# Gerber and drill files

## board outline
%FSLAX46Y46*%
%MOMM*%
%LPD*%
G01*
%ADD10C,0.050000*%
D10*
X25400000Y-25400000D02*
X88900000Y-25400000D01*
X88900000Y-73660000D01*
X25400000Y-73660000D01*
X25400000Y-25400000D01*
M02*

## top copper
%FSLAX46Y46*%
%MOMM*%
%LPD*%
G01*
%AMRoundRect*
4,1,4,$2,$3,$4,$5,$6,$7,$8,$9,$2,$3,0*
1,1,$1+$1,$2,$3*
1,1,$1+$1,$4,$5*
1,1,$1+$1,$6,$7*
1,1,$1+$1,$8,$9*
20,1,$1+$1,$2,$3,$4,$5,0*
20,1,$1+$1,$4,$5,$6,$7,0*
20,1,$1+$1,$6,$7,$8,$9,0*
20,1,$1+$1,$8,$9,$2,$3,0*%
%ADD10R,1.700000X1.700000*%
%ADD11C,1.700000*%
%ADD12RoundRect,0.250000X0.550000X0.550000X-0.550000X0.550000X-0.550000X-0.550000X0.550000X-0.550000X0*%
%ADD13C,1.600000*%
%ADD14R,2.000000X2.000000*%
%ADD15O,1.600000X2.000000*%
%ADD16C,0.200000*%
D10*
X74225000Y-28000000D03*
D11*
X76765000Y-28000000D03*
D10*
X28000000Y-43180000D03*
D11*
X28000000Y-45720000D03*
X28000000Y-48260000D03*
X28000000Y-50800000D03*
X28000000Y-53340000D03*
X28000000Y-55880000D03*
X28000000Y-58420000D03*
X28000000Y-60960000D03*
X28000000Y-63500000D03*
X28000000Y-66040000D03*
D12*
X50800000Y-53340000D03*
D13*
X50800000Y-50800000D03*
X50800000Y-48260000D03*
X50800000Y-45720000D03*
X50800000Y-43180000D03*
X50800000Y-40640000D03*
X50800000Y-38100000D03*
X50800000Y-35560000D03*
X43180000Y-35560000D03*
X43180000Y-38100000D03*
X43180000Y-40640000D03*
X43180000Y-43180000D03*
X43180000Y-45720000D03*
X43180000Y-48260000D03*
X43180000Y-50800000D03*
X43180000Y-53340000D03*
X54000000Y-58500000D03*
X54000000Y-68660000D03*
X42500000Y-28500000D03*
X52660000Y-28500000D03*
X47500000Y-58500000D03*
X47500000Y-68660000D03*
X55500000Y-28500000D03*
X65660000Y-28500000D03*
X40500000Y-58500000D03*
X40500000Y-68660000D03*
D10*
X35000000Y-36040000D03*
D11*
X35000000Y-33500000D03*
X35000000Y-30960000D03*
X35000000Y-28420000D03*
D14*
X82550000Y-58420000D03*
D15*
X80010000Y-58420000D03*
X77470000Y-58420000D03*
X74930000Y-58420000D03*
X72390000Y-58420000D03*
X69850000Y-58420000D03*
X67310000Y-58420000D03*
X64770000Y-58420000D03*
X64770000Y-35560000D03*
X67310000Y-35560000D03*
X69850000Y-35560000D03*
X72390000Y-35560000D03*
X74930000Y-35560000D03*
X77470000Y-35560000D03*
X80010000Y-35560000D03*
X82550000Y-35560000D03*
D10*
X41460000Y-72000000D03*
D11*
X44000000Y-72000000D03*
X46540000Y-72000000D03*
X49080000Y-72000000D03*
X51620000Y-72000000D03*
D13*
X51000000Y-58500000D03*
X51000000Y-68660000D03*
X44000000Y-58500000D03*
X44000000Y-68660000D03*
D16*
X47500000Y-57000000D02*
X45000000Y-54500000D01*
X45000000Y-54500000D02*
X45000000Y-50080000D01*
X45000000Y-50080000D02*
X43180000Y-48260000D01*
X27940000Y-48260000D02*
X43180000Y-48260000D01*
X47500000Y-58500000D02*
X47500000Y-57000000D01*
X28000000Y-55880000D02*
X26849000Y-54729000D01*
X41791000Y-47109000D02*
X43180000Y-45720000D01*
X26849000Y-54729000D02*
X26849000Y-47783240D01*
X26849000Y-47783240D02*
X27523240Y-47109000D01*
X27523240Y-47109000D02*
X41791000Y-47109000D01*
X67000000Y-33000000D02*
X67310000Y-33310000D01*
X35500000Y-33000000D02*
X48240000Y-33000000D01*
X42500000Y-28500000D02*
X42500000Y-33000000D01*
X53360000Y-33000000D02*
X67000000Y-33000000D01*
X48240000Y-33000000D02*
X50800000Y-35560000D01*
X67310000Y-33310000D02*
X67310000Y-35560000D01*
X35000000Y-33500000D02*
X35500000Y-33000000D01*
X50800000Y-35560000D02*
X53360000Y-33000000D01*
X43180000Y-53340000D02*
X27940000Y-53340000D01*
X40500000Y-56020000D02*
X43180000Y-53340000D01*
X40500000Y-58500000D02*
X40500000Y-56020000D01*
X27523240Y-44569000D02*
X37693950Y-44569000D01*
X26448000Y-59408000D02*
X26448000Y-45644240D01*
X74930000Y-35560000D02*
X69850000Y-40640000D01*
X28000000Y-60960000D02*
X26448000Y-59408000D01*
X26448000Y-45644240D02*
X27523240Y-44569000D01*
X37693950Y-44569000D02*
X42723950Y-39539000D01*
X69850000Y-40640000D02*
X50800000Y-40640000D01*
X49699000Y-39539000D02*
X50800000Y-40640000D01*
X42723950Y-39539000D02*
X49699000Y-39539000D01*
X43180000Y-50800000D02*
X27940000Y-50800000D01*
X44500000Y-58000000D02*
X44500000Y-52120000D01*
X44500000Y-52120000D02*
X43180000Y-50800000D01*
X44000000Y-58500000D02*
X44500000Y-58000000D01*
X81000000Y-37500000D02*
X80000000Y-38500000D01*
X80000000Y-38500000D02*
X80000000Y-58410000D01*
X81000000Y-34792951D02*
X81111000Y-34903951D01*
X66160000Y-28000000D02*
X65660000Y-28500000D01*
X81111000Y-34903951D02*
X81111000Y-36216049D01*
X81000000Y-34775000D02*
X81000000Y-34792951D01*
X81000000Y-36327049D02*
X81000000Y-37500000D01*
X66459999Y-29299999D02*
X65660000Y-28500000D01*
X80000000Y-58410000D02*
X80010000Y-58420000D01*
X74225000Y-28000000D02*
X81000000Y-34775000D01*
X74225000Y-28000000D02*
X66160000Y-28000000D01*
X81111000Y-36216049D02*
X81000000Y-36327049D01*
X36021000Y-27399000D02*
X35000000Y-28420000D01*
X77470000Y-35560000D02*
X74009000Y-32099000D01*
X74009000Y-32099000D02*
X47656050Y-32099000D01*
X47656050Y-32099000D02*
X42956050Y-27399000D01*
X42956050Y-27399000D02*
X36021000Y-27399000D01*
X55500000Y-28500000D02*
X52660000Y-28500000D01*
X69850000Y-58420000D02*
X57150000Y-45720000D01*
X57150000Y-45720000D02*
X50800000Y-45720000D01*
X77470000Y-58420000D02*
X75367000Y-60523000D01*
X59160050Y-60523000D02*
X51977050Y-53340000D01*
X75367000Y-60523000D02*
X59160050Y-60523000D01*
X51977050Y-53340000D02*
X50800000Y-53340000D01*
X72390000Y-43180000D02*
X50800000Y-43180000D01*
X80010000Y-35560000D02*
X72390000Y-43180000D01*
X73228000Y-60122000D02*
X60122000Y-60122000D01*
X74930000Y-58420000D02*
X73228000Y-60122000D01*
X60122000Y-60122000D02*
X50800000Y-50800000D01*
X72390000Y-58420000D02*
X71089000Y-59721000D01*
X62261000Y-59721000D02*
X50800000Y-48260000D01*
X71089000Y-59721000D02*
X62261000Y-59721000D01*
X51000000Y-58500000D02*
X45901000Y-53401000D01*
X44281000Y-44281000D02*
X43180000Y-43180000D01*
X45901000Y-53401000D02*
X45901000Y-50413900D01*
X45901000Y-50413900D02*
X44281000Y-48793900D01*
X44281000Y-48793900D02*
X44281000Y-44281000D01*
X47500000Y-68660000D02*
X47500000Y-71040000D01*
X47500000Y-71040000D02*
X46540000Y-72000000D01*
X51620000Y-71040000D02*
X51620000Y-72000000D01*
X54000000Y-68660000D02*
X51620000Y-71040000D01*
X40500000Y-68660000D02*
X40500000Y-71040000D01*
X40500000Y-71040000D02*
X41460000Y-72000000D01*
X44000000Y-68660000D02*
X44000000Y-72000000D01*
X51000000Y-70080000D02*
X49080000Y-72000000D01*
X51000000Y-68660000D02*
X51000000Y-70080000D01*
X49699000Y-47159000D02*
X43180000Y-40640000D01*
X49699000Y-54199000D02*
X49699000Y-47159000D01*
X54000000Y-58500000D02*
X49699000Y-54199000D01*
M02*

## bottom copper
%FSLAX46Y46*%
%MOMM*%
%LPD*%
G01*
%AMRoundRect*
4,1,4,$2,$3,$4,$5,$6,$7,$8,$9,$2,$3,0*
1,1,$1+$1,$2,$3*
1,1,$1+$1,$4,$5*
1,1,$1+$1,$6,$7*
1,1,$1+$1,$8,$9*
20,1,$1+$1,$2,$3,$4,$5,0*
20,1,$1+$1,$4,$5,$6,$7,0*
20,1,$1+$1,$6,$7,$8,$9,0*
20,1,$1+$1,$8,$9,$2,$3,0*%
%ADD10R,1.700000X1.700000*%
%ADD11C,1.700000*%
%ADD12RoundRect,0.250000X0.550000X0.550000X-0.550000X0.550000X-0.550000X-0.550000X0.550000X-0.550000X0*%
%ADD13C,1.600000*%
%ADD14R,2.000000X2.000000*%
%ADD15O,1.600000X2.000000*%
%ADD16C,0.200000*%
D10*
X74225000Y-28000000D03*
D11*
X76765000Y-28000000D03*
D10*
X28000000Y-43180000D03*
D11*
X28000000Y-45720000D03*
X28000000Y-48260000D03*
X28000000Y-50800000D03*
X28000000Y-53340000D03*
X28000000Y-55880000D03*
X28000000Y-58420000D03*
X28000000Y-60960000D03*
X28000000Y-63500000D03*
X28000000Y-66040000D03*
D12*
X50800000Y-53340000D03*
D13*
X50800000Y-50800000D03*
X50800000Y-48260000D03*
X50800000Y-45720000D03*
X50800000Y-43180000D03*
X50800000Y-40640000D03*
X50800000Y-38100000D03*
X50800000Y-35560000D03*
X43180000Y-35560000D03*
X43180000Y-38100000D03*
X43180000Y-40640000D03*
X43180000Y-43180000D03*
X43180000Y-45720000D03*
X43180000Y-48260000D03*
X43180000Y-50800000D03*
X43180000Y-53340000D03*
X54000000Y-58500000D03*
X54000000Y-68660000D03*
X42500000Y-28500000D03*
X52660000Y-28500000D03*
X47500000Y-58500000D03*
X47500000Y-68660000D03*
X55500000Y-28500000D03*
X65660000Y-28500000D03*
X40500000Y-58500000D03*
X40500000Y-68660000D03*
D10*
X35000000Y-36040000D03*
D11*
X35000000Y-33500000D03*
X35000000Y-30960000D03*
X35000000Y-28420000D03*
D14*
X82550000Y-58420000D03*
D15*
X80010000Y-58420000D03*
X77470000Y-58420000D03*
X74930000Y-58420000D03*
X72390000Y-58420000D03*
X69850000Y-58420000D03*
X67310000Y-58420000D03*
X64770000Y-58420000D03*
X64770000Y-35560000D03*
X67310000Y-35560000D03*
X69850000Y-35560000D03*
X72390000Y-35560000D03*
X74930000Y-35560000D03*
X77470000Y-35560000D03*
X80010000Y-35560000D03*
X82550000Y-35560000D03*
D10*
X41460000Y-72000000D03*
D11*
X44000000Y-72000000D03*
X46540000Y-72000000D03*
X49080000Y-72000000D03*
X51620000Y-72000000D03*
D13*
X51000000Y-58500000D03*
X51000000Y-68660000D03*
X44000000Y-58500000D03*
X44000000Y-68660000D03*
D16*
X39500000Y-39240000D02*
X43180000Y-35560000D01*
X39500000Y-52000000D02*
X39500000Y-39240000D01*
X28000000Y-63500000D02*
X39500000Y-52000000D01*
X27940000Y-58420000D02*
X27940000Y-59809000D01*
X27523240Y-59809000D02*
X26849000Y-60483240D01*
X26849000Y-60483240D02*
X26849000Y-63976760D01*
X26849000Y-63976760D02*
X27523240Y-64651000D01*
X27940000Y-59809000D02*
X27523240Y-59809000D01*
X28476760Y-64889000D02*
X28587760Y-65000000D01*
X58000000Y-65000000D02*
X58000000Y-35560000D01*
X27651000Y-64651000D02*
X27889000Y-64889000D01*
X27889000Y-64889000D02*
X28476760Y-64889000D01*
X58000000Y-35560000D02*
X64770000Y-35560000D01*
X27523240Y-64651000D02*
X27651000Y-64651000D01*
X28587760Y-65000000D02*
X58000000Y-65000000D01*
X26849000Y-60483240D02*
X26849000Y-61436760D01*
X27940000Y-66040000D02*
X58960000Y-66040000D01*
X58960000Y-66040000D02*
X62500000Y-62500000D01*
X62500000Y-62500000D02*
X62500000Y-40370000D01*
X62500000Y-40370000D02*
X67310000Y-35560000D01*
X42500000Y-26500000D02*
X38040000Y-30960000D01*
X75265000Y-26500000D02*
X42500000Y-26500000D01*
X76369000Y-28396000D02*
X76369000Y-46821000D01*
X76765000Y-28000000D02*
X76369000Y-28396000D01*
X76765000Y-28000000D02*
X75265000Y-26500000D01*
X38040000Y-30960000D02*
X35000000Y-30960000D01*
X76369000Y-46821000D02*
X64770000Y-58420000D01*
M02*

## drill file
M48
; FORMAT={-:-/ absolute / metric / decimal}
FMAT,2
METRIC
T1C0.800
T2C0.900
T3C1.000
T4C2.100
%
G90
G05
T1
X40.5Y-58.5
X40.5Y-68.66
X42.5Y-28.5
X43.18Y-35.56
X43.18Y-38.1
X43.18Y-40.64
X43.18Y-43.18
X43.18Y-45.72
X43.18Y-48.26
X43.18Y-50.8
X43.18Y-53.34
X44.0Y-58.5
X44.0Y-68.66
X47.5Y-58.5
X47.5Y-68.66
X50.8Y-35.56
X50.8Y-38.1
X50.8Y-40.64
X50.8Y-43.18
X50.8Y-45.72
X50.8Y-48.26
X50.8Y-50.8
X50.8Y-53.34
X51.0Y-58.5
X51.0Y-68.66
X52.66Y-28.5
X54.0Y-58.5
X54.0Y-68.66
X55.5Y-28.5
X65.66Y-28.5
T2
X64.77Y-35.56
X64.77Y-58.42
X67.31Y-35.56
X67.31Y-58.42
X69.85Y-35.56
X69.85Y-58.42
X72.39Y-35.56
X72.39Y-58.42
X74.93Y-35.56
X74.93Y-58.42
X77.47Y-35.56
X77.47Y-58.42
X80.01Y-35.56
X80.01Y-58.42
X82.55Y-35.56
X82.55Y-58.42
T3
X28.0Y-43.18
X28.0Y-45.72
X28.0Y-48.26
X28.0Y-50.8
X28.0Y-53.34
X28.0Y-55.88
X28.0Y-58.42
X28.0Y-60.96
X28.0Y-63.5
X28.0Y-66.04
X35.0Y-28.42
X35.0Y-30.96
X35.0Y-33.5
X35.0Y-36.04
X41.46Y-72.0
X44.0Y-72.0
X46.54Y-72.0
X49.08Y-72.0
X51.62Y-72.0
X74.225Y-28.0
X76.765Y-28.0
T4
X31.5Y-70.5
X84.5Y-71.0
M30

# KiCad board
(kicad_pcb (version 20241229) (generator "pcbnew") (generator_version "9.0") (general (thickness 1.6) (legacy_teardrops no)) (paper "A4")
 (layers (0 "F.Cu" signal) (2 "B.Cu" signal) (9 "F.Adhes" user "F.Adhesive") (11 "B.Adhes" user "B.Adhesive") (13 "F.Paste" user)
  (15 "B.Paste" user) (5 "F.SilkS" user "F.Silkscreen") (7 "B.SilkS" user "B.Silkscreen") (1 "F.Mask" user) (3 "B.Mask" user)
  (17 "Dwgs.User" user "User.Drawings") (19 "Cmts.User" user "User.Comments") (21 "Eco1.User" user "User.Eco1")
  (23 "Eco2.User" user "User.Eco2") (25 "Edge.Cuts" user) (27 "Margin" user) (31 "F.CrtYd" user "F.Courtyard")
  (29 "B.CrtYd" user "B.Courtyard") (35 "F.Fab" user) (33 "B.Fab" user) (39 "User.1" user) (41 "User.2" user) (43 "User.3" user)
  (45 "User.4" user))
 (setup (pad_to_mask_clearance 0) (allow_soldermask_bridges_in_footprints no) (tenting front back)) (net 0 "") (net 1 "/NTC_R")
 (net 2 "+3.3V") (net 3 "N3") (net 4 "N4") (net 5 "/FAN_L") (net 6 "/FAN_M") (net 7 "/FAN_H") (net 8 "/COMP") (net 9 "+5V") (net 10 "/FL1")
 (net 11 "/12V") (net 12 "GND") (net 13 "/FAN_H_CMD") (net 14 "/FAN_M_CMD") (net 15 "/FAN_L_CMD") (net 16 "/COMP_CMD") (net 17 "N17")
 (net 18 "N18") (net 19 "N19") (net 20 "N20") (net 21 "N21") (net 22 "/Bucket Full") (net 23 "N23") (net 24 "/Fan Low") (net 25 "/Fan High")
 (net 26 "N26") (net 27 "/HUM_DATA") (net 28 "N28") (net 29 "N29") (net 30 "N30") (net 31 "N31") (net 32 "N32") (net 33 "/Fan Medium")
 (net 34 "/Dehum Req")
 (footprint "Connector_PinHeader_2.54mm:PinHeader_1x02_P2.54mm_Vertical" (layer "F.Cu") (at 74.225 28 90)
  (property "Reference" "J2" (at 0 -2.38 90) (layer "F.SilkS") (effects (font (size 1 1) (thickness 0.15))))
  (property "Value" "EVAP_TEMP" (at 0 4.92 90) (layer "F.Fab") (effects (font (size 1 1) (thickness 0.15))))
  (pad "1" thru_hole rect (at 0 0 90) (size 1.7 1.7) (drill 1) (layers "*.Cu" "*.Mask") (remove_unused_layers no) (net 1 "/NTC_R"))
  (pad "2" thru_hole circle (at 0 2.54 90) (size 1.7 1.7) (drill 1) (layers "*.Cu" "*.Mask") (remove_unused_layers no) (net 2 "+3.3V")))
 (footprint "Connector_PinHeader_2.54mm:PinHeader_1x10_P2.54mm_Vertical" (layer "F.Cu") (at 28 43.18)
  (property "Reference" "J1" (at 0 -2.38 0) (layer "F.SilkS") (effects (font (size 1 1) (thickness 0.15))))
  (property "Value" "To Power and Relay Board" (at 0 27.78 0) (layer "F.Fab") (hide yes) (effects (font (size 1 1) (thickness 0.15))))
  (pad "1" thru_hole rect (at 0 0) (size 1.7 1.7) (drill 1) (layers "*.Cu" "*.Mask") (remove_unused_layers no) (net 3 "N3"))
  (pad "2" thru_hole circle (at 0 2.54) (size 1.7 1.7) (drill 1) (layers "*.Cu" "*.Mask") (remove_unused_layers no) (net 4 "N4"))
  (pad "3" thru_hole circle (at 0 5.08) (size 1.7 1.7) (drill 1) (layers "*.Cu" "*.Mask") (remove_unused_layers no) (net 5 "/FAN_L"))
  (pad "4" thru_hole circle (at 0 7.62) (size 1.7 1.7) (drill 1) (layers "*.Cu" "*.Mask") (remove_unused_layers no) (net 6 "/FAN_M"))
  (pad "5" thru_hole circle (at 0 10.16) (size 1.7 1.7) (drill 1) (layers "*.Cu" "*.Mask") (remove_unused_layers no) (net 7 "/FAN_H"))
  (pad "6" thru_hole circle (at 0 12.7) (size 1.7 1.7) (drill 1) (layers "*.Cu" "*.Mask") (remove_unused_layers no) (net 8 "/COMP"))
  (pad "7" thru_hole circle (at 0 15.24) (size 1.7 1.7) (drill 1) (layers "*.Cu" "*.Mask") (remove_unused_layers no) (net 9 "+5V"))
  (pad "8" thru_hole circle (at 0 17.78) (size 1.7 1.7) (drill 1) (layers "*.Cu" "*.Mask") (remove_unused_layers no) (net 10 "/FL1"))
  (pad "9" thru_hole circle (at 0 20.32) (size 1.7 1.7) (drill 1) (layers "*.Cu" "*.Mask") (remove_unused_layers no) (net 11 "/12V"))
  (pad "10" thru_hole circle (at 0 22.86) (size 1.7 1.7) (drill 1) (layers "*.Cu" "*.Mask") (remove_unused_layers no) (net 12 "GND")))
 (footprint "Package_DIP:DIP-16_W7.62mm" (layer "F.Cu") (at 50.8 53.34 180)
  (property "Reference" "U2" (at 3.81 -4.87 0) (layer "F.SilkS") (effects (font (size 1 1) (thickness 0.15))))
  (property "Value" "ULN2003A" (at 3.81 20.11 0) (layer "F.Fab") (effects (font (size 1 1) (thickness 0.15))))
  (pad "1" thru_hole roundrect (at 0 0 180) (size 1.6 1.6) (drill 0.8) (layers "*.Cu" "*.Mask") (remove_unused_layers no)
   (roundrect_rratio 0.15625) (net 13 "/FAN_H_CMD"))
  (pad "2" thru_hole circle (at 0 2.54 180) (size 1.6 1.6) (drill 0.8) (layers "*.Cu" "*.Mask") (remove_unused_layers no)
   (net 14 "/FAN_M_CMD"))
  (pad "3" thru_hole circle (at 0 5.08 180) (size 1.6 1.6) (drill 0.8) (layers "*.Cu" "*.Mask") (remove_unused_layers no)
   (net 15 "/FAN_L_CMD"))
  (pad "4" thru_hole circle (at 0 7.62 180) (size 1.6 1.6) (drill 0.8) (layers "*.Cu" "*.Mask") (remove_unused_layers no)
   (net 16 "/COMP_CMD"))
  (pad "5" thru_hole circle (at 0 10.16 180) (size 1.6 1.6) (drill 0.8) (layers "*.Cu" "*.Mask") (remove_unused_layers no) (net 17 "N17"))
  (pad "6" thru_hole circle (at 0 12.7 180) (size 1.6 1.6) (drill 0.8) (layers "*.Cu" "*.Mask") (remove_unused_layers no) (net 10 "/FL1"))
  (pad "7" thru_hole circle (at 0 15.24 180) (size 1.6 1.6) (drill 0.8) (layers "*.Cu" "*.Mask") (remove_unused_layers no) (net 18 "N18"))
  (pad "8" thru_hole circle (at 0 17.78 180) (size 1.6 1.6) (drill 0.8) (layers "*.Cu" "*.Mask") (remove_unused_layers no) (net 12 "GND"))
  (pad "9" thru_hole circle (at 7.62 17.78 180) (size 1.6 1.6) (drill 0.8) (layers "*.Cu" "*.Mask") (remove_unused_layers no)
   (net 11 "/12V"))
  (pad "10" thru_hole circle (at 7.62 15.24 180) (size 1.6 1.6) (drill 0.8) (layers "*.Cu" "*.Mask") (remove_unused_layers no)
   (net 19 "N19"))
  (pad "11" thru_hole circle (at 7.62 12.7 180) (size 1.6 1.6) (drill 0.8) (layers "*.Cu" "*.Mask") (remove_unused_layers no) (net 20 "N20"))
  (pad "12" thru_hole circle (at 7.62 10.16 180) (size 1.6 1.6) (drill 0.8) (layers "*.Cu" "*.Mask") (remove_unused_layers no)
   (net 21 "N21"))
  (pad "13" thru_hole circle (at 7.62 7.62 180) (size 1.6 1.6) (drill 0.8) (layers "*.Cu" "*.Mask") (remove_unused_layers no)
   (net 8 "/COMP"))
  (pad "14" thru_hole circle (at 7.62 5.08 180) (size 1.6 1.6) (drill 0.8) (layers "*.Cu" "*.Mask") (remove_unused_layers no)
   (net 5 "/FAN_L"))
  (pad "15" thru_hole circle (at 7.62 2.54 180) (size 1.6 1.6) (drill 0.8) (layers "*.Cu" "*.Mask") (remove_unused_layers no)
   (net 6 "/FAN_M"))
  (pad "16" thru_hole circle (at 7.62 0 180) (size 1.6 1.6) (drill 0.8) (layers "*.Cu" "*.Mask") (remove_unused_layers no) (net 7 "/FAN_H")))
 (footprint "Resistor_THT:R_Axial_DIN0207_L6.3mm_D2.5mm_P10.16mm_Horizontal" (layer "F.Cu") (at 54 58.5 -90)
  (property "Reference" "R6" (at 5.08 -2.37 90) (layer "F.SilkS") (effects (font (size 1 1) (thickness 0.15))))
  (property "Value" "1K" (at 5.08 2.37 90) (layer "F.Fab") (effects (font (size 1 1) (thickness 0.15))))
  (pad "1" thru_hole circle (at 0 0 270) (size 1.6 1.6) (drill 0.8) (layers "*.Cu" "*.Mask") (remove_unused_layers no) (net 20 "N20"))
  (pad "2" thru_hole circle (at 10.16 0 270) (size 1.6 1.6) (drill 0.8) (layers "*.Cu" "*.Mask") (remove_unused_layers no)
   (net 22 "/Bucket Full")))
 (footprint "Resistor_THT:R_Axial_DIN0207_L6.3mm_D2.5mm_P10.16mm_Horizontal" (layer "F.Cu") (at 42.5 28.5)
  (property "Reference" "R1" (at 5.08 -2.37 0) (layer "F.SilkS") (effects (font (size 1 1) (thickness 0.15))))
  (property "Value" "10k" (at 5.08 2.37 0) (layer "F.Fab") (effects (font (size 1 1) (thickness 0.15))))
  (pad "1" thru_hole circle (at 0 0) (size 1.6 1.6) (drill 0.8) (layers "*.Cu" "*.Mask") (remove_unused_layers no) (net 12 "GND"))
  (pad "2" thru_hole circle (at 10.16 0) (size 1.6 1.6) (drill 0.8) (layers "*.Cu" "*.Mask") (remove_unused_layers no) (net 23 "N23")))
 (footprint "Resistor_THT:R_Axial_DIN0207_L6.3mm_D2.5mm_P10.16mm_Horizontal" (layer "F.Cu") (at 47.5 58.5 -90)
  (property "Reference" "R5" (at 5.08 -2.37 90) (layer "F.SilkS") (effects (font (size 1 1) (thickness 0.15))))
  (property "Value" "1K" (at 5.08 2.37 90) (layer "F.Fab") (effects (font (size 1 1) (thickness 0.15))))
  (pad "1" thru_hole circle (at 0 0 270) (size 1.6 1.6) (drill 0.8) (layers "*.Cu" "*.Mask") (remove_unused_layers no) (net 5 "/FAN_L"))
  (pad "2" thru_hole circle (at 10.16 0 270) (size 1.6 1.6) (drill 0.8) (layers "*.Cu" "*.Mask") (remove_unused_layers no)
   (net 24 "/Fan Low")))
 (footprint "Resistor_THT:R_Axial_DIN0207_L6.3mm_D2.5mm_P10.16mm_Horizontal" (layer "F.Cu") (at 55.5 28.5)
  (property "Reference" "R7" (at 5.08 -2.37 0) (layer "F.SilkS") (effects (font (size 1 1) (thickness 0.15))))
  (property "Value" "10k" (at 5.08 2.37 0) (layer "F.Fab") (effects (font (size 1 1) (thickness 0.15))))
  (pad "1" thru_hole circle (at 0 0) (size 1.6 1.6) (drill 0.8) (layers "*.Cu" "*.Mask") (remove_unused_layers no) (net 23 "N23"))
  (pad "2" thru_hole circle (at 10.16 0) (size 1.6 1.6) (drill 0.8) (layers "*.Cu" "*.Mask") (remove_unused_layers no) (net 1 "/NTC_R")))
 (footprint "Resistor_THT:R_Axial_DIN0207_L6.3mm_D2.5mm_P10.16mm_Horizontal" (layer "F.Cu") (at 40.5 58.5 -90)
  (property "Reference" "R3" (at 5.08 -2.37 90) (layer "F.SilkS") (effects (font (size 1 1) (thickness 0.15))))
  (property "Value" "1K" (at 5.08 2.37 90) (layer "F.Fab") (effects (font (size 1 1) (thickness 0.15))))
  (pad "1" thru_hole circle (at 0 0 270) (size 1.6 1.6) (drill 0.8) (layers "*.Cu" "*.Mask") (remove_unused_layers no) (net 7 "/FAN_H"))
  (pad "2" thru_hole circle (at 10.16 0 270) (size 1.6 1.6) (drill 0.8) (layers "*.Cu" "*.Mask") (remove_unused_layers no)
   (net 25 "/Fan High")))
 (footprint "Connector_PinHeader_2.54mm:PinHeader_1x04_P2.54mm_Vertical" (layer "F.Cu") (at 35 36.04 180)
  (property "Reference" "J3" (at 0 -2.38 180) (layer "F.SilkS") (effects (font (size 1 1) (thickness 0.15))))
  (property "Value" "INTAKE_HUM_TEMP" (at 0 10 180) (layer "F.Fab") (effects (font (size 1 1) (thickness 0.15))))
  (pad "1" thru_hole rect (at 0 0 180) (size 1.7 1.7) (drill 1) (layers "*.Cu" "*.Mask") (remove_unused_layers no) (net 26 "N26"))
  (pad "2" thru_hole circle (at 0 2.54 180) (size 1.7 1.7) (drill 1) (layers "*.Cu" "*.Mask") (remove_unused_layers no) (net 12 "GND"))
  (pad "3" thru_hole circle (at 0 5.08 180) (size 1.7 1.7) (drill 1) (layers "*.Cu" "*.Mask") (remove_unused_layers no) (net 2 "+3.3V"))
  (pad "4" thru_hole circle (at 0 7.62 180) (size 1.7 1.7) (drill 1) (layers "*.Cu" "*.Mask") (remove_unused_layers no) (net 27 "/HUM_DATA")))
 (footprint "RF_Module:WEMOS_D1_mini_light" (layer "F.Cu") (at 64.55 58.42 90)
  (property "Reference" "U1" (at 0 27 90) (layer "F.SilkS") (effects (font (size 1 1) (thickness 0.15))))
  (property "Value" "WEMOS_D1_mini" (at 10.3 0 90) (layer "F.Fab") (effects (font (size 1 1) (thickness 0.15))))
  (pad "1" thru_hole rect (at 0 18 90) (size 2 2) (drill 0.9) (layers "*.Cu" "*.Mask") (remove_unused_layers no) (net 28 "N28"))
  (pad "2" thru_hole oval (at 0 15.46 90) (size 2 1.6) (drill 0.9) (layers "*.Cu" "*.Mask") (remove_unused_layers no) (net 1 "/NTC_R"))
  (pad "3" thru_hole oval (at 0 12.92 90) (size 2 1.6) (drill 0.9) (layers "*.Cu" "*.Mask") (remove_unused_layers no) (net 13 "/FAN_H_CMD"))
  (pad "4" thru_hole oval (at 0 10.38 90) (size 2 1.6) (drill 0.9) (layers "*.Cu" "*.Mask") (remove_unused_layers no) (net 14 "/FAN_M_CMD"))
  (pad "5" thru_hole oval (at 0 7.84 90) (size 2 1.6) (drill 0.9) (layers "*.Cu" "*.Mask") (remove_unused_layers no) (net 15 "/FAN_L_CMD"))
  (pad "6" thru_hole oval (at 0 5.3 90) (size 2 1.6) (drill 0.9) (layers "*.Cu" "*.Mask") (remove_unused_layers no) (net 16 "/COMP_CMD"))
  (pad "7" thru_hole oval (at 0 2.76 90) (size 2 1.6) (drill 0.9) (layers "*.Cu" "*.Mask") (remove_unused_layers no) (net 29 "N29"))
  (pad "8" thru_hole oval (at 0 0.22 90) (size 2 1.6) (drill 0.9) (layers "*.Cu" "*.Mask") (remove_unused_layers no) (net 2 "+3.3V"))
  (pad "9" thru_hole oval (at 22.86 0.22 90) (size 2 1.6) (drill 0.9) (layers "*.Cu" "*.Mask") (remove_unused_layers no) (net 9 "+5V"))
  (pad "10" thru_hole oval (at 22.86 2.76 90) (size 2 1.6) (drill 0.9) (layers "*.Cu" "*.Mask") (remove_unused_layers no) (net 12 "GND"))
  (pad "11" thru_hole oval (at 22.86 5.3 90) (size 2 1.6) (drill 0.9) (layers "*.Cu" "*.Mask") (remove_unused_layers no) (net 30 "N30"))
  (pad "12" thru_hole oval (at 22.86 7.84 90) (size 2 1.6) (drill 0.9) (layers "*.Cu" "*.Mask") (remove_unused_layers no) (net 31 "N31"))
  (pad "13" thru_hole oval (at 22.86 10.38 90) (size 2 1.6) (drill 0.9) (layers "*.Cu" "*.Mask") (remove_unused_layers no) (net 10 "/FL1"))
  (pad "14" thru_hole oval (at 22.86 12.92 90) (size 2 1.6) (drill 0.9) (layers "*.Cu" "*.Mask") (remove_unused_layers no)
   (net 27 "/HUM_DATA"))
  (pad "15" thru_hole oval (at 22.86 15.46 90) (size 2 1.6) (drill 0.9) (layers "*.Cu" "*.Mask") (remove_unused_layers no) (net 17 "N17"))
  (pad "16" thru_hole oval (at 22.86 18 90) (size 2 1.6) (drill 0.9) (layers "*.Cu" "*.Mask") (remove_unused_layers no) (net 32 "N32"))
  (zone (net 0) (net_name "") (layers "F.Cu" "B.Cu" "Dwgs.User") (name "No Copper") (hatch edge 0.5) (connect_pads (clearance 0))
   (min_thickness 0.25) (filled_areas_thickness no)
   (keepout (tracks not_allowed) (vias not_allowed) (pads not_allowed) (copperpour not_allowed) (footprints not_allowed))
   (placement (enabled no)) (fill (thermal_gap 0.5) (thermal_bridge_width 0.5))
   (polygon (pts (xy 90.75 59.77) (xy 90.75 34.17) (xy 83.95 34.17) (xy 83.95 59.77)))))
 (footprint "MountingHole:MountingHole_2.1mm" (layer "F.Cu") (at 84.5 71)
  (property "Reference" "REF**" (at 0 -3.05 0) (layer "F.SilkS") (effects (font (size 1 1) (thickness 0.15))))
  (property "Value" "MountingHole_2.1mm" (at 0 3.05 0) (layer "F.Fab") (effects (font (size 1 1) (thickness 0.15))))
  (pad "" np_thru_hole circle (at 0 0) (size 2.1 2.1) (drill 2.1) (layers "*.Cu" "*.Mask")))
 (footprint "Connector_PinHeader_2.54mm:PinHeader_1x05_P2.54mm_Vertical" (layer "F.Cu") (at 41.46 72 90)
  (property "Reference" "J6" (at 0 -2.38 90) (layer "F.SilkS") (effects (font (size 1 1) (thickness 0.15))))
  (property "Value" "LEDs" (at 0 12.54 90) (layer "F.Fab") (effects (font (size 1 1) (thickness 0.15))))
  (pad "1" thru_hole rect (at 0 0 90) (size 1.7 1.7) (drill 1) (layers "*.Cu" "*.Mask") (remove_unused_layers no) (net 25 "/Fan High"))
  (pad "2" thru_hole circle (at 0 2.54 90) (size 1.7 1.7) (drill 1) (layers "*.Cu" "*.Mask") (remove_unused_layers no)
   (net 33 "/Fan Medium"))
  (pad "3" thru_hole circle (at 0 5.08 90) (size 1.7 1.7) (drill 1) (layers "*.Cu" "*.Mask") (remove_unused_layers no) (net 24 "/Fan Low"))
  (pad "4" thru_hole circle (at 0 7.62 90) (size 1.7 1.7) (drill 1) (layers "*.Cu" "*.Mask") (remove_unused_layers no) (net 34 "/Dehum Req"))
  (pad "5" thru_hole circle (at 0 10.16 90) (size 1.7 1.7) (drill 1) (layers "*.Cu" "*.Mask") (remove_unused_layers no)
   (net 22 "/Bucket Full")))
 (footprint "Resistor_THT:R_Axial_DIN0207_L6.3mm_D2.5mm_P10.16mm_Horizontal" (layer "F.Cu") (at 51 58.5 -90)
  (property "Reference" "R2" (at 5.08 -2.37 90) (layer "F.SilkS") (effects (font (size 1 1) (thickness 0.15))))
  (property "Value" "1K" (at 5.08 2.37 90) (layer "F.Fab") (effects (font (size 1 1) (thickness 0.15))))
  (pad "1" thru_hole circle (at 0 0 270) (size 1.6 1.6) (drill 0.8) (layers "*.Cu" "*.Mask") (remove_unused_layers no) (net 21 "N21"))
  (pad "2" thru_hole circle (at 10.16 0 270) (size 1.6 1.6) (drill 0.8) (layers "*.Cu" "*.Mask") (remove_unused_layers no)
   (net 34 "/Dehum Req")))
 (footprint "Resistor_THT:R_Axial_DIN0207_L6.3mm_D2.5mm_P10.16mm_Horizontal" (layer "F.Cu") (at 44 58.5 -90)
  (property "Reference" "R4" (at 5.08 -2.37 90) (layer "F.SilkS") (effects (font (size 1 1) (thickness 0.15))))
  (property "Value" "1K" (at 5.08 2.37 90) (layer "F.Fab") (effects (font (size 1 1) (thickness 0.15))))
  (pad "1" thru_hole circle (at 0 0 270) (size 1.6 1.6) (drill 0.8) (layers "*.Cu" "*.Mask") (remove_unused_layers no) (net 6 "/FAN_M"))
  (pad "2" thru_hole circle (at 10.16 0 270) (size 1.6 1.6) (drill 0.8) (layers "*.Cu" "*.Mask") (remove_unused_layers no)
   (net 33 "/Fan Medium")))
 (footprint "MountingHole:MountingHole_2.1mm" (layer "F.Cu") (at 31.5 70.5)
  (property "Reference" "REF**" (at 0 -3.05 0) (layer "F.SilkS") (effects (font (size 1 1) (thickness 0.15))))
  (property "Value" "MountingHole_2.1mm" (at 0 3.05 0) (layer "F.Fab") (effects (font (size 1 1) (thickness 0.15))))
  (pad "" np_thru_hole circle (at 0 0) (size 2.1 2.1) (drill 2.1) (layers "*.Cu" "*.Mask")))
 (gr_rect (start 25.4 25.4) (end 88.9 73.66) (stroke (width 0.05) (type solid)) (fill no) (locked yes) (layer "Edge.Cuts"))
 (segment (start 47.5 57) (end 45 54.5) (width 0.2) (layer "F.Cu") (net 5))
 (segment (start 45 54.5) (end 45 50.08) (width 0.2) (layer "F.Cu") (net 5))
 (segment (start 45 50.08) (end 43.18 48.26) (width 0.2) (layer "F.Cu") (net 5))
 (segment (start 27.94 48.26) (end 43.18 48.26) (width 0.2) (layer "F.Cu") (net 5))
 (segment (start 47.5 58.5) (end 47.5 57) (width 0.2) (layer "F.Cu") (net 5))
 (segment (start 39.5 39.24) (end 43.18 35.56) (width 0.2) (layer "B.Cu") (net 11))
 (segment (start 39.5 52) (end 39.5 39.24) (width 0.2) (layer "B.Cu") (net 11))
 (segment (start 28 63.5) (end 39.5 52) (width 0.2) (layer "B.Cu") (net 11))
 (segment (start 28 55.88) (end 26.849 54.729) (width 0.2) (layer "F.Cu") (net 8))
 (segment (start 41.791 47.109) (end 43.18 45.72) (width 0.2) (layer "F.Cu") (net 8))
 (segment (start 26.849 54.729) (end 26.849 47.78324) (width 0.2) (layer "F.Cu") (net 8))
 (segment (start 26.849 47.78324) (end 27.52324 47.109) (width 0.2) (layer "F.Cu") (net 8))
 (segment (start 27.52324 47.109) (end 41.791 47.109) (width 0.2) (layer "F.Cu") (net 8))
 (segment (start 27.94 58.42) (end 27.94 59.809) (width 0.2) (layer "B.Cu") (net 9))
 (segment (start 27.52324 59.809) (end 26.849 60.48324) (width 0.2) (layer "B.Cu") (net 9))
 (segment (start 26.849 60.48324) (end 26.849 63.97676) (width 0.2) (layer "B.Cu") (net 9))
 (segment (start 26.849 63.97676) (end 27.52324 64.651) (width 0.2) (layer "B.Cu") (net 9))
 (segment (start 27.94 59.809) (end 27.52324 59.809) (width 0.2) (layer "B.Cu") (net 9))
 (segment (start 28.47676 64.889) (end 28.58776 65) (width 0.2) (layer "B.Cu") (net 9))
 (segment (start 58 65) (end 58 35.56) (width 0.2) (layer "B.Cu") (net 9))
 (segment (start 27.651 64.651) (end 27.889 64.889) (width 0.2) (layer "B.Cu") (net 9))
 (segment (start 27.889 64.889) (end 28.47676 64.889) (width 0.2) (layer "B.Cu") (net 9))
 (segment (start 58 35.56) (end 64.77 35.56) (width 0.2) (layer "B.Cu") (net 9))
 (segment (start 27.52324 64.651) (end 27.651 64.651) (width 0.2) (layer "B.Cu") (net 9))
 (segment (start 28.58776 65) (end 58 65) (width 0.2) (layer "B.Cu") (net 9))
 (segment (start 26.849 60.48324) (end 26.849 61.43676) (width 0.2) (layer "B.Cu") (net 9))
 (segment (start 67 33) (end 67.31 33.31) (width 0.2) (layer "F.Cu") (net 12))
 (segment (start 35.5 33) (end 48.24 33) (width 0.2) (layer "F.Cu") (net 12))
 (segment (start 42.5 28.5) (end 42.5 33) (width 0.2) (layer "F.Cu") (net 12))
 (segment (start 53.36 33) (end 67 33) (width 0.2) (layer "F.Cu") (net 12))
 (segment (start 48.24 33) (end 50.8 35.56) (width 0.2) (layer "F.Cu") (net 12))
 (segment (start 67.31 33.31) (end 67.31 35.56) (width 0.2) (layer "F.Cu") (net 12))
 (segment (start 35 33.5) (end 35.5 33) (width 0.2) (layer "F.Cu") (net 12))
 (segment (start 50.8 35.56) (end 53.36 33) (width 0.2) (layer "F.Cu") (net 12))
 (segment (start 27.94 66.04) (end 58.96 66.04) (width 0.2) (layer "B.Cu") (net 12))
 (segment (start 58.96 66.04) (end 62.5 62.5) (width 0.2) (layer "B.Cu") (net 12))
 (segment (start 62.5 62.5) (end 62.5 40.37) (width 0.2) (layer "B.Cu") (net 12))
 (segment (start 62.5 40.37) (end 67.31 35.56) (width 0.2) (layer "B.Cu") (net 12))
 (segment (start 43.18 53.34) (end 27.94 53.34) (width 0.2) (layer "F.Cu") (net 7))
 (segment (start 40.5 56.02) (end 43.18 53.34) (width 0.2) (layer "F.Cu") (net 7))
 (segment (start 40.5 58.5) (end 40.5 56.02) (width 0.2) (layer "F.Cu") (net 7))
 (segment (start 27.52324 44.569) (end 37.69395 44.569) (width 0.2) (layer "F.Cu") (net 10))
 (segment (start 26.448 59.408) (end 26.448 45.64424) (width 0.2) (layer "F.Cu") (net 10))
 (segment (start 74.93 35.56) (end 69.85 40.64) (width 0.2) (layer "F.Cu") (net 10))
 (segment (start 28 60.96) (end 26.448 59.408) (width 0.2) (layer "F.Cu") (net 10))
 (segment (start 26.448 45.64424) (end 27.52324 44.569) (width 0.2) (layer "F.Cu") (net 10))
 (segment (start 37.69395 44.569) (end 42.72395 39.539) (width 0.2) (layer "F.Cu") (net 10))
 (segment (start 69.85 40.64) (end 50.8 40.64) (width 0.2) (layer "F.Cu") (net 10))
 (segment (start 49.699 39.539) (end 50.8 40.64) (width 0.2) (layer "F.Cu") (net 10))
 (segment (start 42.72395 39.539) (end 49.699 39.539) (width 0.2) (layer "F.Cu") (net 10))
 (segment (start 43.18 50.8) (end 27.94 50.8) (width 0.2) (layer "F.Cu") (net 6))
 (segment (start 44.5 58) (end 44.5 52.12) (width 0.2) (layer "F.Cu") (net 6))
 (segment (start 44.5 52.12) (end 43.18 50.8) (width 0.2) (layer "F.Cu") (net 6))
 (segment (start 44 58.5) (end 44.5 58) (width 0.2) (layer "F.Cu") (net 6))
 (segment (start 81 37.5) (end 80 38.5) (width 0.2) (layer "F.Cu") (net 1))
 (segment (start 80 38.5) (end 80 58.41) (width 0.2) (layer "F.Cu") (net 1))
 (segment (start 81 34.792951) (end 81.111 34.903951) (width 0.2) (layer "F.Cu") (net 1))
 (segment (start 66.16 28) (end 65.66 28.5) (width 0.2) (layer "F.Cu") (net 1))
 (segment (start 81.111 34.903951) (end 81.111 36.216049) (width 0.2) (layer "F.Cu") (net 1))
 (segment (start 81 34.775) (end 81 34.792951) (width 0.2) (layer "F.Cu") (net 1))
 (segment (start 81 36.327049) (end 81 37.5) (width 0.2) (layer "F.Cu") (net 1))
 (segment (start 66.459999 29.299999) (end 65.66 28.5) (width 0.2) (layer "F.Cu") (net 1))
 (segment (start 80 58.41) (end 80.01 58.42) (width 0.2) (layer "F.Cu") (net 1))
 (segment (start 74.225 28) (end 81 34.775) (width 0.2) (layer "F.Cu") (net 1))
 (segment (start 74.225 28) (end 66.16 28) (width 0.2) (layer "F.Cu") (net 1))
 (segment (start 81.111 36.216049) (end 81 36.327049) (width 0.2) (layer "F.Cu") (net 1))
 (segment (start 36.021 27.399) (end 35 28.42) (width 0.2) (layer "F.Cu") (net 27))
 (segment (start 77.47 35.56) (end 74.009 32.099) (width 0.2) (layer "F.Cu") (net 27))
 (segment (start 74.009 32.099) (end 47.65605 32.099) (width 0.2) (layer "F.Cu") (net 27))
 (segment (start 47.65605 32.099) (end 42.95605 27.399) (width 0.2) (layer "F.Cu") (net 27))
 (segment (start 42.95605 27.399) (end 36.021 27.399) (width 0.2) (layer "F.Cu") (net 27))
 (segment (start 42.5 26.5) (end 38.04 30.96) (width 0.2) (layer "B.Cu") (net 2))
 (segment (start 75.265 26.5) (end 42.5 26.5) (width 0.2) (layer "B.Cu") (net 2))
 (segment (start 76.369 28.396) (end 76.369 46.821) (width 0.2) (layer "B.Cu") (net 2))
 (segment (start 76.765 28) (end 76.369 28.396) (width 0.2) (layer "B.Cu") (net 2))
 (segment (start 76.765 28) (end 75.265 26.5) (width 0.2) (layer "B.Cu") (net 2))
 (segment (start 38.04 30.96) (end 35 30.96) (width 0.2) (layer "B.Cu") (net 2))
 (segment (start 76.369 46.821) (end 64.77 58.42) (width 0.2) (layer "B.Cu") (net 2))
 (segment (start 55.5 28.5) (end 52.66 28.5) (width 0.2) (layer "F.Cu") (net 23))
 (segment (start 69.85 58.42) (end 57.15 45.72) (width 0.2) (layer "F.Cu") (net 16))
 (segment (start 57.15 45.72) (end 50.8 45.72) (width 0.2) (layer "F.Cu") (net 16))
 (segment (start 77.47 58.42) (end 75.367 60.523) (width 0.2) (layer "F.Cu") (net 13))
 (segment (start 59.16005 60.523) (end 51.97705 53.34) (width 0.2) (layer "F.Cu") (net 13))
 (segment (start 75.367 60.523) (end 59.16005 60.523) (width 0.2) (layer "F.Cu") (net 13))
 (segment (start 51.97705 53.34) (end 50.8 53.34) (width 0.2) (layer "F.Cu") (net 13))
 (segment (start 72.39 43.18) (end 50.8 43.18) (width 0.2) (layer "F.Cu") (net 17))
 (segment (start 80.01 35.56) (end 72.39 43.18) (width 0.2) (layer "F.Cu") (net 17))
 (segment (start 73.228 60.122) (end 60.122 60.122) (width 0.2) (layer "F.Cu") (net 14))
 (segment (start 74.93 58.42) (end 73.228 60.122) (width 0.2) (layer "F.Cu") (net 14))
 (segment (start 60.122 60.122) (end 50.8 50.8) (width 0.2) (layer "F.Cu") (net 14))
 (segment (start 72.39 58.42) (end 71.089 59.721) (width 0.2) (layer "F.Cu") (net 15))
 (segment (start 62.261 59.721) (end 50.8 48.26) (width 0.2) (layer "F.Cu") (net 15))
 (segment (start 71.089 59.721) (end 62.261 59.721) (width 0.2) (layer "F.Cu") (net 15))
 (segment (start 51 58.5) (end 45.901 53.401) (width 0.2) (layer "F.Cu") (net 21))
 (segment (start 44.281 44.281) (end 43.18 43.18) (width 0.2) (layer "F.Cu") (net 21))
 (segment (start 45.901 53.401) (end 45.901 50.4139) (width 0.2) (layer "F.Cu") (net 21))
 (segment (start 45.901 50.4139) (end 44.281 48.7939) (width 0.2) (layer "F.Cu") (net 21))
 (segment (start 44.281 48.7939) (end 44.281 44.281) (width 0.2) (layer "F.Cu") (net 21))
 (segment (start 47.5 68.66) (end 47.5 71.04) (width 0.2) (layer "F.Cu") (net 24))
 (segment (start 47.5 71.04) (end 46.54 72) (width 0.2) (layer "F.Cu") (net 24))
 (segment (start 51.62 71.04) (end 51.62 72) (width 0.2) (layer "F.Cu") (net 22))
 (segment (start 54 68.66) (end 51.62 71.04) (width 0.2) (layer "F.Cu") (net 22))
 (segment (start 40.5 68.66) (end 40.5 71.04) (width 0.2) (layer "F.Cu") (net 25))
 (segment (start 40.5 71.04) (end 41.46 72) (width 0.2) (layer "F.Cu") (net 25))
 (segment (start 44 68.66) (end 44 72) (width 0.2) (layer "F.Cu") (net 33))
 (segment (start 51 70.08) (end 49.08 72) (width 0.2) (layer "F.Cu") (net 34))
 (segment (start 51 68.66) (end 51 70.08) (width 0.2) (layer "F.Cu") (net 34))
 (segment (start 49.699 47.159) (end 43.18 40.64) (width 0.2) (layer "F.Cu") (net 20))
 (segment (start 49.699 54.199) (end 49.699 47.159) (width 0.2) (layer "F.Cu") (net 20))
 (segment (start 54 58.5) (end 49.699 54.199) (width 0.2) (layer "F.Cu") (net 20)))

